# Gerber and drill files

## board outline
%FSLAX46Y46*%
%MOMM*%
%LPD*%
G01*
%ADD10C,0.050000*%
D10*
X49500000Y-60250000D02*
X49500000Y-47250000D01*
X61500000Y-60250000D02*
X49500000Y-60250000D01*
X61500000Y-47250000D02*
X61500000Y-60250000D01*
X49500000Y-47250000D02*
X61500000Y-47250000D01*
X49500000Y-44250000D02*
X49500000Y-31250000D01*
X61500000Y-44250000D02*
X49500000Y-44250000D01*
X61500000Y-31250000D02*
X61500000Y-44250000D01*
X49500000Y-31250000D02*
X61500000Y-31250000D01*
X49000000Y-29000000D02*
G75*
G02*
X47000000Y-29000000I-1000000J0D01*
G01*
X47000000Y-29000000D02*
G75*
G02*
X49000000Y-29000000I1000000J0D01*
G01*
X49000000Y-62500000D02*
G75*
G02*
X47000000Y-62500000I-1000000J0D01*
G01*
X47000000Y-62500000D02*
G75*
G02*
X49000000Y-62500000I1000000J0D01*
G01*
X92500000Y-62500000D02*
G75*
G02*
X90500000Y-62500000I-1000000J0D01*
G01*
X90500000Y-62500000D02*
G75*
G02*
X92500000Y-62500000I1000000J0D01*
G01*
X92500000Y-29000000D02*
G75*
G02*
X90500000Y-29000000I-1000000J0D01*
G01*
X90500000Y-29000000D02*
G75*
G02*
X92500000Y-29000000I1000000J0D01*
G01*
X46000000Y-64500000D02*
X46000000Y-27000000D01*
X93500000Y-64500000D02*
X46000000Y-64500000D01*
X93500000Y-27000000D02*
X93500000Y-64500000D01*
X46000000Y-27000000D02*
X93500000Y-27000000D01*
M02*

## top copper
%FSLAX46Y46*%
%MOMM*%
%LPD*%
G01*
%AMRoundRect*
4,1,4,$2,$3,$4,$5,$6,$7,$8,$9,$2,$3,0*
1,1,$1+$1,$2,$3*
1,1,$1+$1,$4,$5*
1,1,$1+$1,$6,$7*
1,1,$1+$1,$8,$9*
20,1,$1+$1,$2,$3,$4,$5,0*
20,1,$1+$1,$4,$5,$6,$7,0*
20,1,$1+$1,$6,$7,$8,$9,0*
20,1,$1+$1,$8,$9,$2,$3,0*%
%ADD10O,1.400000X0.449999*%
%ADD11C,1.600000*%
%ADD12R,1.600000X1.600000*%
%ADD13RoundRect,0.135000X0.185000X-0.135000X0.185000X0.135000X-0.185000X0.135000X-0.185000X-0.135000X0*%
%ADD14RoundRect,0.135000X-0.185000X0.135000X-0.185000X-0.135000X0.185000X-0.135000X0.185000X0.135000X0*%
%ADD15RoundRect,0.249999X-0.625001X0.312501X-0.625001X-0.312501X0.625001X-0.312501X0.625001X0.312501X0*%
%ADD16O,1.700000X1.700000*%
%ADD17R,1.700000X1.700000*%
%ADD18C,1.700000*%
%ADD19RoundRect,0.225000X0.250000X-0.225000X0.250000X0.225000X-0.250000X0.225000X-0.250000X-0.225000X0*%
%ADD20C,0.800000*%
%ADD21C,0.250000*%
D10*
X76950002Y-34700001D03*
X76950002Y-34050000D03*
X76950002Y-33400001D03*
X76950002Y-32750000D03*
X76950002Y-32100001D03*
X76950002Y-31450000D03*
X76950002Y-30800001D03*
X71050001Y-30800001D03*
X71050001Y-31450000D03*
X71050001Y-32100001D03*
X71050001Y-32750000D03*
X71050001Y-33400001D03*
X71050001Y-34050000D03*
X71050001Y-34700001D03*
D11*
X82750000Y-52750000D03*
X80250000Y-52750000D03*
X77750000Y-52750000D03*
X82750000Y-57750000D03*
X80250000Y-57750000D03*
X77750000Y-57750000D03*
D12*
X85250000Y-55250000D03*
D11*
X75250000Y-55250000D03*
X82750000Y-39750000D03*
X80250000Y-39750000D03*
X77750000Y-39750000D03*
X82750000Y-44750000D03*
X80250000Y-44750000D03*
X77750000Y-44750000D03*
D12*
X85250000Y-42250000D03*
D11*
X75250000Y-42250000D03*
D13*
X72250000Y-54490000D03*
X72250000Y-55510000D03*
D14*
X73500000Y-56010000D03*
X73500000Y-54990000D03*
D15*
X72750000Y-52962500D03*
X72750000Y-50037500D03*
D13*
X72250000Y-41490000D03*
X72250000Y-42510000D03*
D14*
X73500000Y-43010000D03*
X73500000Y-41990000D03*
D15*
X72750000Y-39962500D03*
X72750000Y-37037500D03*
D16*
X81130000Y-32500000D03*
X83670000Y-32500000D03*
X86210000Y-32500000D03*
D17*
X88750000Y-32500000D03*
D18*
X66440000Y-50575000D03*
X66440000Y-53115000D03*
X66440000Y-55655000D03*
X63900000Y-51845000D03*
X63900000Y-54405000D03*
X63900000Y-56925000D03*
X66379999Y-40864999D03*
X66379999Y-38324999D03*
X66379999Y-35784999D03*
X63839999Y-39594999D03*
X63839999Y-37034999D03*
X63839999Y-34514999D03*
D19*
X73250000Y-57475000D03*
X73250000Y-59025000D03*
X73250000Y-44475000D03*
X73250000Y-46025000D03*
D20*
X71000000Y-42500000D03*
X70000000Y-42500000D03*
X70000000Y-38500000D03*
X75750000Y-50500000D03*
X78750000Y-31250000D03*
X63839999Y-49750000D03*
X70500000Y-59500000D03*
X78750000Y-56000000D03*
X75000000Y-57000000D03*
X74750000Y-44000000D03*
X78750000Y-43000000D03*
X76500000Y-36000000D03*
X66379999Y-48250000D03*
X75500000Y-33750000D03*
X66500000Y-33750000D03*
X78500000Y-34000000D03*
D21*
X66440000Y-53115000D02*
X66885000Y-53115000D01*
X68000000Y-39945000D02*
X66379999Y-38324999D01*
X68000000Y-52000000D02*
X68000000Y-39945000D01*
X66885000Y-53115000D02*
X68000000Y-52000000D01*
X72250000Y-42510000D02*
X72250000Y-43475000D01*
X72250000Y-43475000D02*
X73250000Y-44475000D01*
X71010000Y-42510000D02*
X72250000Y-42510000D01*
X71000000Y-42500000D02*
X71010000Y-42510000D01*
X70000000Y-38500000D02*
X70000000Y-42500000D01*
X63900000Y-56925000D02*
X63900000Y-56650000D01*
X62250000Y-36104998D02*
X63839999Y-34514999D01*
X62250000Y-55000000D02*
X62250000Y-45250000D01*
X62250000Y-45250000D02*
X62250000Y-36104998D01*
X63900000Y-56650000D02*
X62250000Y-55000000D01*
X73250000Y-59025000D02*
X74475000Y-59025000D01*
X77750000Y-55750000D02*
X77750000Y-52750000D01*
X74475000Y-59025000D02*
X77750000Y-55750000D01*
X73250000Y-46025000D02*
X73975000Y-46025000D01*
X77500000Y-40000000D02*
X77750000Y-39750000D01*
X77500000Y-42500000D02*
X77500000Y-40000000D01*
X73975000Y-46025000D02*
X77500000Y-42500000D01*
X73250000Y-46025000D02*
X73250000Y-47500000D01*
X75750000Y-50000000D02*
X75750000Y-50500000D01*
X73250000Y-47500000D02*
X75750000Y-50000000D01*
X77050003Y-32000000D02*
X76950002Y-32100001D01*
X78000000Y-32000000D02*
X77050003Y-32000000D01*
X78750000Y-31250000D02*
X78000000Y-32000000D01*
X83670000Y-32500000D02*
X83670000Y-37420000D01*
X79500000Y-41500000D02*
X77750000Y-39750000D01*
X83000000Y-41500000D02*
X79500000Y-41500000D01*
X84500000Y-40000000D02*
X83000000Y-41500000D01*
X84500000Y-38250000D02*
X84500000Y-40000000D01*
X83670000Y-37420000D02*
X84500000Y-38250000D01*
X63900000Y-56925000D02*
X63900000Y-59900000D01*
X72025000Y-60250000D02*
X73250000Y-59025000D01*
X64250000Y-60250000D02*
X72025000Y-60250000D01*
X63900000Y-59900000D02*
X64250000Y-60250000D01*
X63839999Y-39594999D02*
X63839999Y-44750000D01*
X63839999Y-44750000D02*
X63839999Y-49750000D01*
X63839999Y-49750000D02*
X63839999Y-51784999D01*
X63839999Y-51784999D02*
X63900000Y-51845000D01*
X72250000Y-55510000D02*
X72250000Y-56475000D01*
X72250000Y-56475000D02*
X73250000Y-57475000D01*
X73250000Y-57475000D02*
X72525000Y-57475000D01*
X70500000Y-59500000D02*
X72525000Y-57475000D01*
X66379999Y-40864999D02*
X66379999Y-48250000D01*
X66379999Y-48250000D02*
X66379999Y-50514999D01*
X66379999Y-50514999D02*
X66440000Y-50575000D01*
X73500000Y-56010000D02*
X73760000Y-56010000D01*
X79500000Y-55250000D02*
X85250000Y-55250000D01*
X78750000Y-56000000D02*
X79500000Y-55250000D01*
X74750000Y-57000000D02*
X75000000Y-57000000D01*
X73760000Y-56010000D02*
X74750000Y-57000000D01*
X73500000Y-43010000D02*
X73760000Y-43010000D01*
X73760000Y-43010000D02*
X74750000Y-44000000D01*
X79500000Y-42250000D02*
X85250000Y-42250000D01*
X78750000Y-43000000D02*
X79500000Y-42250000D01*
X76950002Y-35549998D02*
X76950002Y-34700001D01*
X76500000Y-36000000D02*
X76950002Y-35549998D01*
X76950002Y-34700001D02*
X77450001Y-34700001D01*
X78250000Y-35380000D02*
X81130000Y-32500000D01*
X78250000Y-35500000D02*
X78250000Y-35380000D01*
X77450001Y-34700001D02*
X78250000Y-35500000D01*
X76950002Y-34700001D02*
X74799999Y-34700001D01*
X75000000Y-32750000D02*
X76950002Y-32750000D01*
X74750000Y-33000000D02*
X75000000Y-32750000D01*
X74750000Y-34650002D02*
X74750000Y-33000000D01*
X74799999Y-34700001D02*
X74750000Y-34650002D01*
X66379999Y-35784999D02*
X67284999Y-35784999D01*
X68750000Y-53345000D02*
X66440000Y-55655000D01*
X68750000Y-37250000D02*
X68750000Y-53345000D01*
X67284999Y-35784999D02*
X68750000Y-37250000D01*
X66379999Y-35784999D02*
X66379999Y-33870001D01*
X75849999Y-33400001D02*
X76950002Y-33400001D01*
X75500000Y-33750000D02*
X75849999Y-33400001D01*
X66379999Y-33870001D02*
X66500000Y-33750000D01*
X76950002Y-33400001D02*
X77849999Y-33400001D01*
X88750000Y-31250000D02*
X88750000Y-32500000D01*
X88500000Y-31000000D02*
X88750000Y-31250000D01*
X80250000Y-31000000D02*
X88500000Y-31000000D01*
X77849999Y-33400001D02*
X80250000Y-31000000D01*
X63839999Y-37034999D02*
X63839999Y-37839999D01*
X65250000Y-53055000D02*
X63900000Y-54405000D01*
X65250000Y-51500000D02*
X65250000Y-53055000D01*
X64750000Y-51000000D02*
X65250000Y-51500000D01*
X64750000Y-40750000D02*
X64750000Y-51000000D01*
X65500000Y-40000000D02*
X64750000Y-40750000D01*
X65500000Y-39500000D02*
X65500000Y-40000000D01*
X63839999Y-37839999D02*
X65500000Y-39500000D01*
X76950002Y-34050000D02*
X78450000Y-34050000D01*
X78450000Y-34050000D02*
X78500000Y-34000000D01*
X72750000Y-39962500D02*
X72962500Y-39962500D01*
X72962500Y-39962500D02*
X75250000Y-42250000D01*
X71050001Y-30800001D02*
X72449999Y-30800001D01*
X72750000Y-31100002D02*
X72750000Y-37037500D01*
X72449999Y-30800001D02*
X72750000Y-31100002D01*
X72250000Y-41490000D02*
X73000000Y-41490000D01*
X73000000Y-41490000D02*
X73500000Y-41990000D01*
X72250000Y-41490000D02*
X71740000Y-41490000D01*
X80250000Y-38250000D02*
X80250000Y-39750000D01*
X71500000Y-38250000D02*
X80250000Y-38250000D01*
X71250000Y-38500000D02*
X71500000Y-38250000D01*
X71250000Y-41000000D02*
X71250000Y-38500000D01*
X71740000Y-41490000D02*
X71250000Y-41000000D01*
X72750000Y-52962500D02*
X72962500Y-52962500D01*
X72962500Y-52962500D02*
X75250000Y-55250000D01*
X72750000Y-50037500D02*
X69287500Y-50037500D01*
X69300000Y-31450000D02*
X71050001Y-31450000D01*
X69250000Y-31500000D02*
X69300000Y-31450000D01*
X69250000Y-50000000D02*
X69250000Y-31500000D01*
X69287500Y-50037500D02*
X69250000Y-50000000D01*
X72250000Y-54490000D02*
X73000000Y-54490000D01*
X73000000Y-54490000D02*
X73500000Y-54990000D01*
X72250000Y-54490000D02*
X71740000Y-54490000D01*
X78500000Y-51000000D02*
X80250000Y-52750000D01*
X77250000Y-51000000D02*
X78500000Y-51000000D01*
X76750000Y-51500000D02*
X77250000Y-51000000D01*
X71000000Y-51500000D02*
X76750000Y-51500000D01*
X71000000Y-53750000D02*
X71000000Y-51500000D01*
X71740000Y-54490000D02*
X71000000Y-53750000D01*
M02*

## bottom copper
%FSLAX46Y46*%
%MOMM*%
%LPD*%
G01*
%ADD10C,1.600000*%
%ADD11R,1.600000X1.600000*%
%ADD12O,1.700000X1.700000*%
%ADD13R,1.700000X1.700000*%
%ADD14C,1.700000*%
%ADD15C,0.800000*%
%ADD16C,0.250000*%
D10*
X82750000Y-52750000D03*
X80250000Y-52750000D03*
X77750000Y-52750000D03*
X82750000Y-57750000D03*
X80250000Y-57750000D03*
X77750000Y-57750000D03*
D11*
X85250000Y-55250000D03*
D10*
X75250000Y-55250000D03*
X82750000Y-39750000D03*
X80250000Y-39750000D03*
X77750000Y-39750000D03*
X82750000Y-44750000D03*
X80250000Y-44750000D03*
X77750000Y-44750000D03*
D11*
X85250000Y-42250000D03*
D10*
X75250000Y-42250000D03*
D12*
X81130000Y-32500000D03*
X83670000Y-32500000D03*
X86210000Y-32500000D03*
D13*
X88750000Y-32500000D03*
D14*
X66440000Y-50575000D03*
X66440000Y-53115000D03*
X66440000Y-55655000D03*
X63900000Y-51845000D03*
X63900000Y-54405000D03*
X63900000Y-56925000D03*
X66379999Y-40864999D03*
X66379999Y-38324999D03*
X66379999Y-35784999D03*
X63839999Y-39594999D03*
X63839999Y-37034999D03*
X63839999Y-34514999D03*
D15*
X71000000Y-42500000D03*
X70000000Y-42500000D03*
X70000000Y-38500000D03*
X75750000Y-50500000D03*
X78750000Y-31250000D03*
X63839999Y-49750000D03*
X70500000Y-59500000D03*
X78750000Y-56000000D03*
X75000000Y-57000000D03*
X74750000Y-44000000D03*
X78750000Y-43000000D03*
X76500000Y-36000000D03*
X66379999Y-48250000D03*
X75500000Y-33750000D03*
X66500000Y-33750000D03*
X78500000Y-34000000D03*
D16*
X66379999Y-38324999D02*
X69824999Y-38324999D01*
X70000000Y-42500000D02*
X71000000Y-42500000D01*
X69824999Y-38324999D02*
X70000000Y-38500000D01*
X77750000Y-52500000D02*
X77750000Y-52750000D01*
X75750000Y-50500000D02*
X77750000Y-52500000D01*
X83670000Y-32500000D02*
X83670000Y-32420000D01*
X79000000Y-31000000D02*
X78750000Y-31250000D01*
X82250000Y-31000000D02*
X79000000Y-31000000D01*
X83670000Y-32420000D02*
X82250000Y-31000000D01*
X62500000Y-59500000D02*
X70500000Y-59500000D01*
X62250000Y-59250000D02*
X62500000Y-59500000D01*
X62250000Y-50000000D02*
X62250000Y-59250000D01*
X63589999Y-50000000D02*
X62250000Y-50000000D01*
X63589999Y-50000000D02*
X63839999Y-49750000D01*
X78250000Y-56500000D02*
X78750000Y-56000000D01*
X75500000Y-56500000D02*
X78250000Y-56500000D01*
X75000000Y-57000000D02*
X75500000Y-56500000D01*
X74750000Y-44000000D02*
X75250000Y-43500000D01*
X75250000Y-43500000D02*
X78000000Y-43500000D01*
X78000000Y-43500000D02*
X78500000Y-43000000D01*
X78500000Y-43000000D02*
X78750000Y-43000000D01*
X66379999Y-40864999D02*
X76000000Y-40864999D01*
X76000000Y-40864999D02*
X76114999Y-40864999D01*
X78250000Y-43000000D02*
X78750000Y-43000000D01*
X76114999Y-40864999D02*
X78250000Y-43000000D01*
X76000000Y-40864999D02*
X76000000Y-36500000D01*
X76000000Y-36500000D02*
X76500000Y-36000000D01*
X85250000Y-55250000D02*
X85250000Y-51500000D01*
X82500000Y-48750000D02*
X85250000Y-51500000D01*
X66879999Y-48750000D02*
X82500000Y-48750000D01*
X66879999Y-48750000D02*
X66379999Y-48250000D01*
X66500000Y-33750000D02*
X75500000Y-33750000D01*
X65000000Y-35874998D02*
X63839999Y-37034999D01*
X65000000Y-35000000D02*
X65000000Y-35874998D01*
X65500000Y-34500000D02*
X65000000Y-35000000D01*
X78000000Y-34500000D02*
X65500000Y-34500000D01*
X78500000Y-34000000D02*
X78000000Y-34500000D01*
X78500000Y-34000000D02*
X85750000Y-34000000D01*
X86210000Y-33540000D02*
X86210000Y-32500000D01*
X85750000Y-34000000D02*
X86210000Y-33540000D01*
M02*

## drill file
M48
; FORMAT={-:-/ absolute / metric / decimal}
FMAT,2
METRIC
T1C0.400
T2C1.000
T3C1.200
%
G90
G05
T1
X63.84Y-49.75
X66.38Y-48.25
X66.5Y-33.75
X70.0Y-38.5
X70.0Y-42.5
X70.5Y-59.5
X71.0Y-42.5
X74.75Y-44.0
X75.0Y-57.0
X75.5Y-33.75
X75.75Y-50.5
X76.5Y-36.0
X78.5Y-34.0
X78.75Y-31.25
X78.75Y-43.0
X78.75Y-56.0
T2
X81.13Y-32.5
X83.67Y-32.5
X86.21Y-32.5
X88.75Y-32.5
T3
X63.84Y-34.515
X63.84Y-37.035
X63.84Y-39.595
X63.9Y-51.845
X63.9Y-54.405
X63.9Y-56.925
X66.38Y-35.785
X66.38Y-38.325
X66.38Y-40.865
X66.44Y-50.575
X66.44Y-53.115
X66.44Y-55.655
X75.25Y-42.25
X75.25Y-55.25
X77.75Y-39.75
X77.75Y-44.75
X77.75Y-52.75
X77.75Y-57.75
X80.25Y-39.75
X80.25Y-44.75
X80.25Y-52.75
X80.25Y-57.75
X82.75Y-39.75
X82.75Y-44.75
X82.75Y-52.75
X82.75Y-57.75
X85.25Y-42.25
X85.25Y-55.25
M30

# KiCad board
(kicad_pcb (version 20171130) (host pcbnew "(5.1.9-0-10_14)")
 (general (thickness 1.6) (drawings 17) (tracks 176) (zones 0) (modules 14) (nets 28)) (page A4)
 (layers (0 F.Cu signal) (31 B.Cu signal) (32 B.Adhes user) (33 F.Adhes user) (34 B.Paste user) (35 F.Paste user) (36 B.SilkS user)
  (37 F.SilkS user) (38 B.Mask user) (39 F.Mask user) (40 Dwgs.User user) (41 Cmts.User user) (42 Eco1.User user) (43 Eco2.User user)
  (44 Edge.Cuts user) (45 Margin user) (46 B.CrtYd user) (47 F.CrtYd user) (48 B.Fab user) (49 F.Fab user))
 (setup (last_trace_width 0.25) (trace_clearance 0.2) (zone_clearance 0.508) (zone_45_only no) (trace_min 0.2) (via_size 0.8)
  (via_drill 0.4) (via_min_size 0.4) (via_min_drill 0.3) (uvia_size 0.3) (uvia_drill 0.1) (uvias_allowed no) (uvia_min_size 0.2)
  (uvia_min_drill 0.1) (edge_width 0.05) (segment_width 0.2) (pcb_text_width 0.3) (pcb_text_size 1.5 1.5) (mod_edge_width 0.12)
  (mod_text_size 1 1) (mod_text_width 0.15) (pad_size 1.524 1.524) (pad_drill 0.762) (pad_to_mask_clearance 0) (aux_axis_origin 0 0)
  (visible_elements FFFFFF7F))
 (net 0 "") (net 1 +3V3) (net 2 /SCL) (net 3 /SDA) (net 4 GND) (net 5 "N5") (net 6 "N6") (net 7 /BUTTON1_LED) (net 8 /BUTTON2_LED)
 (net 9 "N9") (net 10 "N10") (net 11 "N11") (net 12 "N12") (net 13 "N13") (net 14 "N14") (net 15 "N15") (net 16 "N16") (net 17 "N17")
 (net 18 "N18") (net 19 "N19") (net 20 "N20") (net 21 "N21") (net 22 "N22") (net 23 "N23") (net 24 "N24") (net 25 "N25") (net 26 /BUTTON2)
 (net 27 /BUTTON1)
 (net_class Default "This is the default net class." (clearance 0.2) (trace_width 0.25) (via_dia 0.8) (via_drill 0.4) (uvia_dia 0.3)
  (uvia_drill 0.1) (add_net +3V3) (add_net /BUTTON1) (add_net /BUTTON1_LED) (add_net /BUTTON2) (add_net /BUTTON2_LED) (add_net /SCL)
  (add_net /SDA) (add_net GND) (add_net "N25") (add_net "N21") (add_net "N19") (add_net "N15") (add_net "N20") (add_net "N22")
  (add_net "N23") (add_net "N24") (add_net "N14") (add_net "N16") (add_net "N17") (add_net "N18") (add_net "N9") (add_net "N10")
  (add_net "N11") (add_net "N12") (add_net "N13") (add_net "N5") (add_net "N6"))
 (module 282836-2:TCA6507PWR (layer F.Cu) (at 74 32.75 180)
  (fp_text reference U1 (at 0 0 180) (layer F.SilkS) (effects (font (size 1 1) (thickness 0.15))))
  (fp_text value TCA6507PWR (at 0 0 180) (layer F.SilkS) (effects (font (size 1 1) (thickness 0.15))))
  (pad 1 smd oval (at -2.950002 -1.950001 270) (size 0.449999 1.4) (layers F.Cu F.Paste F.Mask) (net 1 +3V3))
  (pad 2 smd oval (at -2.950002 -1.3 270) (size 0.449999 1.4) (layers F.Cu F.Paste F.Mask) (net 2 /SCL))
  (pad 3 smd oval (at -2.950002 -0.650001 270) (size 0.449999 1.4) (layers F.Cu F.Paste F.Mask) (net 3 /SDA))
  (pad 4 smd oval (at -2.950002 0 270) (size 0.449999 1.4) (layers F.Cu F.Paste F.Mask) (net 1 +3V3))
  (pad 5 smd oval (at -2.950002 0.649999 270) (size 0.449999 1.4) (layers F.Cu F.Paste F.Mask) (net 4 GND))
  (pad 6 smd oval (at -2.950002 1.3 270) (size 0.449999 1.4) (layers F.Cu F.Paste F.Mask) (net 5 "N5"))
  (pad 7 smd oval (at -2.950002 1.949999 270) (size 0.449999 1.4) (layers F.Cu F.Paste F.Mask) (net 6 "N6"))
  (pad 8 smd oval (at 2.949999 1.949999 270) (size 0.449999 1.4) (layers F.Cu F.Paste F.Mask) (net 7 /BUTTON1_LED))
  (pad 9 smd oval (at 2.949999 1.3 270) (size 0.449999 1.4) (layers F.Cu F.Paste F.Mask) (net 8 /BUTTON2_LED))
  (pad 10 smd oval (at 2.949999 0.649999 270) (size 0.449999 1.4) (layers F.Cu F.Paste F.Mask) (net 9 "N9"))
  (pad 11 smd oval (at 2.949999 0 270) (size 0.449999 1.4) (layers F.Cu F.Paste F.Mask) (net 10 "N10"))
  (pad 12 smd oval (at 2.949999 -0.650001 270) (size 0.449999 1.4) (layers F.Cu F.Paste F.Mask) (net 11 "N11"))
  (pad 13 smd oval (at 2.949999 -1.3 270) (size 0.449999 1.4) (layers F.Cu F.Paste F.Mask) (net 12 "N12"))
  (pad 14 smd oval (at 2.949999 -1.950001 270) (size 0.449999 1.4) (layers F.Cu F.Paste F.Mask) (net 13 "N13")))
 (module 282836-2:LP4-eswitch (layer F.Cu) (at 80.25 55.25)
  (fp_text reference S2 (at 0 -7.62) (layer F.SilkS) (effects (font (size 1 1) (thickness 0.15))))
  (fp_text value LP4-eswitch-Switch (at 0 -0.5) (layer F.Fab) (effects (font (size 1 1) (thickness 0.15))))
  (pad 1 thru_hole circle (at 2.5 -2.5) (size 1.6 1.6) (drill 1.2) (layers *.Cu *.Mask) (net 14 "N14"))
  (pad 2 thru_hole circle (at 0 -2.5) (size 1.6 1.6) (drill 1.2) (layers *.Cu *.Mask) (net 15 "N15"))
  (pad 3 thru_hole circle (at -2.5 -2.5) (size 1.6 1.6) (drill 1.2) (layers *.Cu *.Mask) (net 4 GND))
  (pad 4 thru_hole circle (at 2.5 2.5) (size 1.6 1.6) (drill 1.2) (layers *.Cu *.Mask) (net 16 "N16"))
  (pad 5 thru_hole circle (at 0 2.5) (size 1.6 1.6) (drill 1.2) (layers *.Cu *.Mask) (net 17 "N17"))
  (pad 6 thru_hole circle (at -2.5 2.5) (size 1.6 1.6) (drill 1.2) (layers *.Cu *.Mask) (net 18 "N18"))
  (pad L1 thru_hole rect (at 5 0) (size 1.6 1.6) (drill 1.2) (layers *.Cu *.Mask) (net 1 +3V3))
  (pad L2 thru_hole circle (at -5 0) (size 1.6 1.6) (drill 1.2) (layers *.Cu *.Mask) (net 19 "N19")))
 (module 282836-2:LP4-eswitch (layer F.Cu) (at 80.25 42.25)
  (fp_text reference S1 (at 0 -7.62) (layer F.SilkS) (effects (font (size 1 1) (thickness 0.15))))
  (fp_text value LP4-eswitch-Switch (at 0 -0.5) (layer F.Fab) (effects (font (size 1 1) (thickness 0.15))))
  (pad 1 thru_hole circle (at 2.5 -2.5) (size 1.6 1.6) (drill 1.2) (layers *.Cu *.Mask) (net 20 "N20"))
  (pad 2 thru_hole circle (at 0 -2.5) (size 1.6 1.6) (drill 1.2) (layers *.Cu *.Mask) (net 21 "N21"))
  (pad 3 thru_hole circle (at -2.5 -2.5) (size 1.6 1.6) (drill 1.2) (layers *.Cu *.Mask) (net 4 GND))
  (pad 4 thru_hole circle (at 2.5 2.5) (size 1.6 1.6) (drill 1.2) (layers *.Cu *.Mask) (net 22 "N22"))
  (pad 5 thru_hole circle (at 0 2.5) (size 1.6 1.6) (drill 1.2) (layers *.Cu *.Mask) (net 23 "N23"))
  (pad 6 thru_hole circle (at -2.5 2.5) (size 1.6 1.6) (drill 1.2) (layers *.Cu *.Mask) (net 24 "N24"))
  (pad L1 thru_hole rect (at 5 0) (size 1.6 1.6) (drill 1.2) (layers *.Cu *.Mask) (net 1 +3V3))
  (pad L2 thru_hole circle (at -5 0) (size 1.6 1.6) (drill 1.2) (layers *.Cu *.Mask) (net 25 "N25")))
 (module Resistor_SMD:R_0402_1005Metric (layer F.Cu) (at 72.25 55 90)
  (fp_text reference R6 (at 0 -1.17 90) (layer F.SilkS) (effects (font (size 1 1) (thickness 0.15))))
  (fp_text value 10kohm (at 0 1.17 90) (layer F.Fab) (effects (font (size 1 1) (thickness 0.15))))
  (pad 2 smd roundrect (at 0.51 0 90) (size 0.54 0.64) (layers F.Cu F.Paste F.Mask) (roundrect_rratio 0.25) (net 15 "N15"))
  (pad 1 smd roundrect (at -0.51 0 90) (size 0.54 0.64) (layers F.Cu F.Paste F.Mask) (roundrect_rratio 0.25) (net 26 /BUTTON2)))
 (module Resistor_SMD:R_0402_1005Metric (layer F.Cu) (at 73.5 55.5 270)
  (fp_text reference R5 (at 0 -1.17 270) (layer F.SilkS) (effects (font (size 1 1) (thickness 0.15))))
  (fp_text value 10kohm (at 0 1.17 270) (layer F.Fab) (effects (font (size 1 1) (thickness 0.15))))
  (pad 2 smd roundrect (at 0.51 0 270) (size 0.54 0.64) (layers F.Cu F.Paste F.Mask) (roundrect_rratio 0.25) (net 1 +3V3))
  (pad 1 smd roundrect (at -0.51 0 270) (size 0.54 0.64) (layers F.Cu F.Paste F.Mask) (roundrect_rratio 0.25) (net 15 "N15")))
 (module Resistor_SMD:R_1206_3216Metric (layer F.Cu) (at 72.75 51.5 270)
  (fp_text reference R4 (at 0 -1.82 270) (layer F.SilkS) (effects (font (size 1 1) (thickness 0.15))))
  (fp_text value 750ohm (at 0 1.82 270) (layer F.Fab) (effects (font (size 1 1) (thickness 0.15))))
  (pad 2 smd roundrect (at 1.4625 0 270) (size 1.125 1.75) (layers F.Cu F.Paste F.Mask) (roundrect_rratio 0.2222213333333333) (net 19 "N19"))
  (pad 1 smd roundrect (at -1.4625 0 270) (size 1.125 1.75) (layers F.Cu F.Paste F.Mask) (roundrect_rratio 0.2222213333333333)
   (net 8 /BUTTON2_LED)))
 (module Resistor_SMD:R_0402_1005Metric (layer F.Cu) (at 72.25 42 90)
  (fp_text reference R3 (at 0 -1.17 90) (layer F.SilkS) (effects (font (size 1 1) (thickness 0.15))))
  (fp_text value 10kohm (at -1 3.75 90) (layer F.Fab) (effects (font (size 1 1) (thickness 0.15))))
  (pad 2 smd roundrect (at 0.51 0 90) (size 0.54 0.64) (layers F.Cu F.Paste F.Mask) (roundrect_rratio 0.25) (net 21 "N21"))
  (pad 1 smd roundrect (at -0.51 0 90) (size 0.54 0.64) (layers F.Cu F.Paste F.Mask) (roundrect_rratio 0.25) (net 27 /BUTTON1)))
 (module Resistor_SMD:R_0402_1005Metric (layer F.Cu) (at 73.5 42.5 270)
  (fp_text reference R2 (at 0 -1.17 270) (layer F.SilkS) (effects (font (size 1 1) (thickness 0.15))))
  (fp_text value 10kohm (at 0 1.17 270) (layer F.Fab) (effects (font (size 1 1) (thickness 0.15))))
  (pad 2 smd roundrect (at 0.51 0 270) (size 0.54 0.64) (layers F.Cu F.Paste F.Mask) (roundrect_rratio 0.25) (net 1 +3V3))
  (pad 1 smd roundrect (at -0.51 0 270) (size 0.54 0.64) (layers F.Cu F.Paste F.Mask) (roundrect_rratio 0.25) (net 21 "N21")))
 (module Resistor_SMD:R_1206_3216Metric (layer F.Cu) (at 72.75 38.5 270)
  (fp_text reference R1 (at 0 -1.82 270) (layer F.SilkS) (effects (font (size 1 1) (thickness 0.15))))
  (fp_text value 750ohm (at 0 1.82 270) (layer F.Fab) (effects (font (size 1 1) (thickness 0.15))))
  (pad 2 smd roundrect (at 1.4625 0 270) (size 1.125 1.75) (layers F.Cu F.Paste F.Mask) (roundrect_rratio 0.2222213333333333) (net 25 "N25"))
  (pad 1 smd roundrect (at -1.4625 0 270) (size 1.125 1.75) (layers F.Cu F.Paste F.Mask) (roundrect_rratio 0.2222213333333333)
   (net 7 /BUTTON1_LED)))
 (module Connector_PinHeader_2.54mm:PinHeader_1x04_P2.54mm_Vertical (layer F.Cu) (at 88.75 32.5 270)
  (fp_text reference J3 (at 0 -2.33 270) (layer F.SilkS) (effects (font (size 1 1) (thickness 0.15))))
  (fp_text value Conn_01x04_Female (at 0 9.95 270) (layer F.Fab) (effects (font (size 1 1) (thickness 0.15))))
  (pad 4 thru_hole oval (at 0 7.62 270) (size 1.7 1.7) (drill 1) (layers *.Cu *.Mask) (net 1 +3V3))
  (pad 3 thru_hole oval (at 0 5.08 270) (size 1.7 1.7) (drill 1) (layers *.Cu *.Mask) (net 4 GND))
  (pad 2 thru_hole oval (at 0 2.54 270) (size 1.7 1.7) (drill 1) (layers *.Cu *.Mask) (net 2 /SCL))
  (pad 1 thru_hole rect (at 0 0 270) (size 1.7 1.7) (drill 1) (layers *.Cu *.Mask) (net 3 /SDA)))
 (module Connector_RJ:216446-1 (layer B.Cu) (at 61.5 53.75 90)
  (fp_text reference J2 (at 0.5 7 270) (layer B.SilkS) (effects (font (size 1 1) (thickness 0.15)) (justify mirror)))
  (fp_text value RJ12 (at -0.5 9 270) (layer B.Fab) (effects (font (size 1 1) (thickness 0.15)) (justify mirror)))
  (pad 6 thru_hole circle (at 3.175 4.94 90) (size 1.7 1.7) (drill 1.2) (layers *.Cu *.Mask) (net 1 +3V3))
  (pad 4 thru_hole circle (at 0.635 4.94 90) (size 1.7 1.7) (drill 1.2) (layers *.Cu *.Mask) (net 27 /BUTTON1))
  (pad 2 thru_hole circle (at -1.905 4.94 90) (size 1.7 1.7) (drill 1.2) (layers *.Cu *.Mask) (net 3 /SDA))
  (pad 5 thru_hole circle (at 1.905 2.4 90) (size 1.7 1.7) (drill 1.2) (layers *.Cu *.Mask) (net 26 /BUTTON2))
  (pad 3 thru_hole circle (at -0.655 2.4 90) (size 1.7 1.7) (drill 1.2) (layers *.Cu *.Mask) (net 2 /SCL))
  (pad 1 thru_hole circle (at -3.175 2.4 90) (size 1.7 1.7) (drill 1.2) (layers *.Cu *.Mask) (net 4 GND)))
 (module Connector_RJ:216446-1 (layer F.Cu) (at 61.439999 37.689999 270)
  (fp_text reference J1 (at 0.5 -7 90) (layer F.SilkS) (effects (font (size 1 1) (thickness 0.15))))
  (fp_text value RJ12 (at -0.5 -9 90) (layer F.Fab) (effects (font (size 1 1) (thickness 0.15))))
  (pad 6 thru_hole circle (at 3.175 -4.94 270) (size 1.7 1.7) (drill 1.2) (layers *.Cu *.Mask) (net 1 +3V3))
  (pad 4 thru_hole circle (at 0.635 -4.94 270) (size 1.7 1.7) (drill 1.2) (layers *.Cu *.Mask) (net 27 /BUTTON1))
  (pad 2 thru_hole circle (at -1.905 -4.94 270) (size 1.7 1.7) (drill 1.2) (layers *.Cu *.Mask) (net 3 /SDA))
  (pad 5 thru_hole circle (at 1.905 -2.4 270) (size 1.7 1.7) (drill 1.2) (layers *.Cu *.Mask) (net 26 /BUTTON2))
  (pad 3 thru_hole circle (at -0.655 -2.4 270) (size 1.7 1.7) (drill 1.2) (layers *.Cu *.Mask) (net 2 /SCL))
  (pad 1 thru_hole circle (at -3.175 -2.4 270) (size 1.7 1.7) (drill 1.2) (layers *.Cu *.Mask) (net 4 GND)))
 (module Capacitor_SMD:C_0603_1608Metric (layer F.Cu) (at 73.25 58.25 90)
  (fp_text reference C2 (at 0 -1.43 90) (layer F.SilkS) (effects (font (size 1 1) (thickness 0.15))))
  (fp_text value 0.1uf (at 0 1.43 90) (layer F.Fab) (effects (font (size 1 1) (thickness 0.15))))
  (pad 2 smd roundrect (at 0.775 0 90) (size 0.9 0.95) (layers F.Cu F.Paste F.Mask) (roundrect_rratio 0.25) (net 26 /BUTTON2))
  (pad 1 smd roundrect (at -0.775 0 90) (size 0.9 0.95) (layers F.Cu F.Paste F.Mask) (roundrect_rratio 0.25) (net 4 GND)))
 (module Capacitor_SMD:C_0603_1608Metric (layer F.Cu) (at 73.25 45.25 90)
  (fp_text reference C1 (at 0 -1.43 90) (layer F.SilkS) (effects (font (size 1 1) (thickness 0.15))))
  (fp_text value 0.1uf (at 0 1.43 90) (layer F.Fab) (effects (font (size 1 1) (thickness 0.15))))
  (pad 2 smd roundrect (at 0.775 0 90) (size 0.9 0.95) (layers F.Cu F.Paste F.Mask) (roundrect_rratio 0.25) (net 27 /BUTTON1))
  (pad 1 smd roundrect (at -0.775 0 90) (size 0.9 0.95) (layers F.Cu F.Paste F.Mask) (roundrect_rratio 0.25) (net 4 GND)))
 (gr_line (start 49.5 60.25) (end 49.5 47.25) (angle 90) (layer Edge.Cuts) (width 0.05))
 (gr_line (start 61.5 60.25) (end 49.5 60.25) (angle 90) (layer Edge.Cuts) (width 0.05))
 (gr_line (start 61.5 47.25) (end 61.5 60.25) (angle 90) (layer Edge.Cuts) (width 0.05))
 (gr_line (start 49.5 47.25) (end 61.5 47.25) (angle 90) (layer Edge.Cuts) (width 0.05))
 (gr_line (start 49.5 44.25) (end 49.5 31.25) (angle 90) (layer Edge.Cuts) (width 0.05))
 (gr_line (start 61.5 44.25) (end 49.5 44.25) (angle 90) (layer Edge.Cuts) (width 0.05))
 (gr_line (start 61.5 31.25) (end 61.5 44.25) (angle 90) (layer Edge.Cuts) (width 0.05))
 (gr_line (start 49.5 31.25) (end 61.5 31.25) (angle 90) (layer Edge.Cuts) (width 0.05))
 (gr_circle (center 48 29) (end 49 29) (layer Edge.Cuts) (width 0.05))
 (gr_circle (center 48 62.5) (end 49 62.5) (layer Edge.Cuts) (width 0.05))
 (gr_circle (center 91.5 62.5) (end 92.5 62.5) (layer Edge.Cuts) (width 0.05))
 (gr_circle (center 91.5 29) (end 92.5 29) (layer Edge.Cuts) (width 0.05))
 (gr_line (start 46 64.5) (end 46 27) (angle 90) (layer Edge.Cuts) (width 0.05))
 (gr_line (start 93.5 64.5) (end 46 64.5) (angle 90) (layer Edge.Cuts) (width 0.05))
 (gr_line (start 93.5 27) (end 93.5 64.5) (angle 90) (layer Edge.Cuts) (width 0.05))
 (gr_line (start 46 27) (end 93.5 27) (angle 90) (layer Edge.Cuts) (width 0.05))
 (segment (start 66.44 53.115) (end 66.885 53.115) (width 0.25) (layer F.Cu) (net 27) (status C00000))
 (segment (start 68 39.945) (end 66.379999 38.324999) (width 0.25) (layer F.Cu) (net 27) (status 800000))
 (segment (start 68 52) (end 68 39.945) (width 0.25) (layer F.Cu) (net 27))
 (segment (start 66.885 53.115) (end 68 52) (width 0.25) (layer F.Cu) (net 27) (status 400000))
 (segment (start 72.25 42.51) (end 72.25 43.475) (width 0.25) (layer F.Cu) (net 27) (status 400000))
 (segment (start 72.25 43.475) (end 73.25 44.475) (width 0.25) (layer F.Cu) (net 27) (status 800000))
 (segment (start 66.379999 38.324999) (end 69.824999 38.324999) (width 0.25) (layer B.Cu) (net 27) (status 400000))
 (segment (start 71.01 42.51) (end 72.25 42.51) (width 0.25) (layer F.Cu) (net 27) (status 800000))
 (segment (start 71 42.5) (end 71.01 42.51) (width 0.25) (layer F.Cu) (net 27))
 (via (at 71 42.5) (size 0.8) (drill 0.4) (layers F.Cu B.Cu) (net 27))
 (segment (start 70 42.5) (end 71 42.5) (width 0.25) (layer B.Cu) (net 27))
 (via (at 70 42.5) (size 0.8) (drill 0.4) (layers F.Cu B.Cu) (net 27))
 (segment (start 70 38.5) (end 70 42.5) (width 0.25) (layer F.Cu) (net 27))
 (via (at 70 38.5) (size 0.8) (drill 0.4) (layers F.Cu B.Cu) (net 27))
 (segment (start 69.824999 38.324999) (end 70 38.5) (width 0.25) (layer B.Cu) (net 27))
 (segment (start 63.9 56.925) (end 63.9 56.65) (width 0.25) (layer F.Cu) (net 4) (status C00000))
 (segment (start 62.25 36.104998) (end 63.839999 34.514999) (width 0.25) (layer F.Cu) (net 4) (status 800000))
 (segment (start 62.25 55) (end 62.25 45.25) (width 0.25) (layer F.Cu) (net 4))
 (segment (start 62.25 45.25) (end 62.25 36.104998) (width 0.25) (layer F.Cu) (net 4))
 (segment (start 63.9 56.65) (end 62.25 55) (width 0.25) (layer F.Cu) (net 4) (status 400000))
 (segment (start 73.25 59.025) (end 74.475 59.025) (width 0.25) (layer F.Cu) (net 4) (status 400000))
 (segment (start 77.75 55.75) (end 77.75 52.75) (width 0.25) (layer F.Cu) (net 4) (status 800000))
 (segment (start 74.475 59.025) (end 77.75 55.75) (width 0.25) (layer F.Cu) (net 4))
 (segment (start 73.25 46.025) (end 73.975 46.025) (width 0.25) (layer F.Cu) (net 4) (status 400000))
 (segment (start 77.5 40) (end 77.75 39.75) (width 0.25) (layer F.Cu) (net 4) (status C00000))
 (segment (start 77.5 42.5) (end 77.5 40) (width 0.25) (layer F.Cu) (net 4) (status 800000))
 (segment (start 73.975 46.025) (end 77.5 42.5) (width 0.25) (layer F.Cu) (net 4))
 (segment (start 73.25 46.025) (end 73.25 47.5) (width 0.25) (layer F.Cu) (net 4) (status 400000))
 (segment (start 77.75 52.5) (end 77.75 52.75) (width 0.25) (layer B.Cu) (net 4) (status C00000))
 (segment (start 75.75 50.5) (end 77.75 52.5) (width 0.25) (layer B.Cu) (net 4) (status 800000))
 (via (at 75.75 50.5) (size 0.8) (drill 0.4) (layers F.Cu B.Cu) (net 4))
 (segment (start 75.75 50) (end 75.75 50.5) (width 0.25) (layer F.Cu) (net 4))
 (segment (start 73.25 47.5) (end 75.75 50) (width 0.25) (layer F.Cu) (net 4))
 (segment (start 83.67 32.5) (end 83.67 32.42) (width 0.25) (layer B.Cu) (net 4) (status C00000))
 (segment (start 77.050003 32) (end 76.950002 32.100001) (width 0.25) (layer F.Cu) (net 4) (status C00000))
 (segment (start 78 32) (end 77.050003 32) (width 0.25) (layer F.Cu) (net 4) (status 800000))
 (segment (start 78.75 31.25) (end 78 32) (width 0.25) (layer F.Cu) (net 4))
 (via (at 78.75 31.25) (size 0.8) (drill 0.4) (layers F.Cu B.Cu) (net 4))
 (segment (start 79 31) (end 78.75 31.25) (width 0.25) (layer B.Cu) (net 4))
 (segment (start 82.25 31) (end 79 31) (width 0.25) (layer B.Cu) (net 4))
 (segment (start 83.67 32.42) (end 82.25 31) (width 0.25) (layer B.Cu) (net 4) (status 400000))
 (segment (start 83.67 32.5) (end 83.67 37.42) (width 0.25) (layer F.Cu) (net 4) (status 400000))
 (segment (start 79.5 41.5) (end 77.75 39.75) (width 0.25) (layer F.Cu) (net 4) (status 800000))
 (segment (start 83 41.5) (end 79.5 41.5) (width 0.25) (layer F.Cu) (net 4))
 (segment (start 84.5 40) (end 83 41.5) (width 0.25) (layer F.Cu) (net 4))
 (segment (start 84.5 38.25) (end 84.5 40) (width 0.25) (layer F.Cu) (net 4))
 (segment (start 83.67 37.42) (end 84.5 38.25) (width 0.25) (layer F.Cu) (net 4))
 (segment (start 63.9 56.925) (end 63.9 59.9) (width 0.25) (layer F.Cu) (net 4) (status 400000))
 (segment (start 72.025 60.25) (end 73.25 59.025) (width 0.25) (layer F.Cu) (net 4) (status 800000))
 (segment (start 64.25 60.25) (end 72.025 60.25) (width 0.25) (layer F.Cu) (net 4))
 (segment (start 63.9 59.9) (end 64.25 60.25) (width 0.25) (layer F.Cu) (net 4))
 (segment (start 63.839999 39.594999) (end 63.839999 44.75) (width 0.25) (layer F.Cu) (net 26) (status 400000))
 (segment (start 63.839999 44.75) (end 63.839999 49.75) (width 0.25) (layer F.Cu) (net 26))
 (segment (start 63.839999 49.75) (end 63.839999 51.784999) (width 0.25) (layer F.Cu) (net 26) (status 800000))
 (segment (start 63.839999 51.784999) (end 63.9 51.845) (width 0.25) (layer F.Cu) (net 26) (status C00000))
 (segment (start 72.25 55.51) (end 72.25 56.475) (width 0.25) (layer F.Cu) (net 26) (status 400000))
 (segment (start 72.25 56.475) (end 73.25 57.475) (width 0.25) (layer F.Cu) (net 26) (status 800000))
 (via (at 63.839999 49.75) (size 0.8) (drill 0.4) (layers F.Cu B.Cu) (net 26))
 (segment (start 73.25 57.475) (end 72.525 57.475) (width 0.25) (layer F.Cu) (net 26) (status 400000))
 (segment (start 70.5 59.5) (end 72.525 57.475) (width 0.25) (layer F.Cu) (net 26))
 (via (at 70.5 59.5) (size 0.8) (drill 0.4) (layers F.Cu B.Cu) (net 26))
 (segment (start 62.5 59.5) (end 70.5 59.5) (width 0.25) (layer B.Cu) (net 26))
 (segment (start 62.25 59.25) (end 62.5 59.5) (width 0.25) (layer B.Cu) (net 26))
 (segment (start 62.25 50) (end 62.25 59.25) (width 0.25) (layer B.Cu) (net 26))
 (segment (start 63.589999 50) (end 62.25 50) (width 0.25) (layer B.Cu) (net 26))
 (segment (start 63.589999 50) (end 63.839999 49.75) (width 0.25) (layer B.Cu) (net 26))
 (segment (start 66.379999 40.864999) (end 66.379999 48.25) (width 0.25) (layer F.Cu) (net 1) (status 400000))
 (segment (start 66.379999 48.25) (end 66.379999 50.514999) (width 0.25) (layer F.Cu) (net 1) (status 800000))
 (segment (start 66.379999 50.514999) (end 66.44 50.575) (width 0.25) (layer F.Cu) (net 1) (status C00000))
 (segment (start 73.5 56.01) (end 73.76 56.01) (width 0.25) (layer F.Cu) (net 1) (status C00000))
 (segment (start 79.5 55.25) (end 85.25 55.25) (width 0.25) (layer F.Cu) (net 1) (status 800000))
 (segment (start 78.75 56) (end 79.5 55.25) (width 0.25) (layer F.Cu) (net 1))
 (via (at 78.75 56) (size 0.8) (drill 0.4) (layers F.Cu B.Cu) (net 1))
 (segment (start 78.25 56.5) (end 78.75 56) (width 0.25) (layer B.Cu) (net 1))
 (segment (start 75.5 56.5) (end 78.25 56.5) (width 0.25) (layer B.Cu) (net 1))
 (segment (start 75 57) (end 75.5 56.5) (width 0.25) (layer B.Cu) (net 1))
 (via (at 75 57) (size 0.8) (drill 0.4) (layers F.Cu B.Cu) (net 1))
 (segment (start 74.75 57) (end 75 57) (width 0.25) (layer F.Cu) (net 1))
 (segment (start 73.76 56.01) (end 74.75 57) (width 0.25) (layer F.Cu) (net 1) (status 400000))
 (segment (start 73.5 43.01) (end 73.76 43.01) (width 0.25) (layer F.Cu) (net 1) (status C00000))
 (segment (start 73.76 43.01) (end 74.75 44) (width 0.25) (layer F.Cu) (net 1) (status 400000))
 (via (at 74.75 44) (size 0.8) (drill 0.4) (layers F.Cu B.Cu) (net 1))
 (segment (start 74.75 44) (end 75.25 43.5) (width 0.25) (layer B.Cu) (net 1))
 (segment (start 75.25 43.5) (end 78 43.5) (width 0.25) (layer B.Cu) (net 1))
 (segment (start 78 43.5) (end 78.5 43) (width 0.25) (layer B.Cu) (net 1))
 (segment (start 78.5 43) (end 78.75 43) (width 0.25) (layer B.Cu) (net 1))
 (segment (start 79.5 42.25) (end 85.25 42.25) (width 0.25) (layer F.Cu) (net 1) (status 800000))
 (via (at 78.75 43) (size 0.8) (drill 0.4) (layers F.Cu B.Cu) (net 1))
 (segment (start 78.75 43) (end 79.5 42.25) (width 0.25) (layer F.Cu) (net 1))
 (segment (start 66.379999 40.864999) (end 76 40.864999) (width 0.25) (layer B.Cu) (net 1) (status 400000))
 (segment (start 76 40.864999) (end 76.114999 40.864999) (width 0.25) (layer B.Cu) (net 1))
 (segment (start 78.25 43) (end 78.75 43) (width 0.25) (layer B.Cu) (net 1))
 (segment (start 76.114999 40.864999) (end 78.25 43) (width 0.25) (layer B.Cu) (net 1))
 (segment (start 76 40.864999) (end 76 36.5) (width 0.25) (layer B.Cu) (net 1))
 (segment (start 76.950002 35.549998) (end 76.950002 34.700001) (width 0.25) (layer F.Cu) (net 1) (status 800000))
 (segment (start 76.5 36) (end 76.950002 35.549998) (width 0.25) (layer F.Cu) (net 1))
 (via (at 76.5 36) (size 0.8) (drill 0.4) (layers F.Cu B.Cu) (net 1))
 (segment (start 76 36.5) (end 76.5 36) (width 0.25) (layer B.Cu) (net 1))
 (segment (start 76.950002 34.700001) (end 77.450001 34.700001) (width 0.25) (layer F.Cu) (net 1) (status C00000))
 (segment (start 78.25 35.38) (end 81.13 32.5) (width 0.25) (layer F.Cu) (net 1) (status 800000))
 (segment (start 78.25 35.5) (end 78.25 35.38) (width 0.25) (layer F.Cu) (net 1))
 (segment (start 77.450001 34.700001) (end 78.25 35.5) (width 0.25) (layer F.Cu) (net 1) (status 400000))
 (segment (start 76.950002 34.700001) (end 74.799999 34.700001) (width 0.25) (layer F.Cu) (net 1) (status 400000))
 (segment (start 75 32.75) (end 76.950002 32.75) (width 0.25) (layer F.Cu) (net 1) (status 800000))
 (segment (start 74.75 33) (end 75 32.75) (width 0.25) (layer F.Cu) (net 1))
 (segment (start 74.75 34.650002) (end 74.75 33) (width 0.25) (layer F.Cu) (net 1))
 (segment (start 74.799999 34.700001) (end 74.75 34.650002) (width 0.25) (layer F.Cu) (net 1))
 (via (at 66.379999 48.25) (size 0.8) (drill 0.4) (layers F.Cu B.Cu) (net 1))
 (segment (start 85.25 55.25) (end 85.25 51.5) (width 0.25) (layer B.Cu) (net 1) (status 400000))
 (segment (start 82.5 48.75) (end 85.25 51.5) (width 0.25) (layer B.Cu) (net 1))
 (segment (start 66.879999 48.75) (end 82.5 48.75) (width 0.25) (layer B.Cu) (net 1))
 (segment (start 66.879999 48.75) (end 66.379999 48.25) (width 0.25) (layer B.Cu) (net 1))
 (segment (start 66.379999 35.784999) (end 67.284999 35.784999) (width 0.25) (layer F.Cu) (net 3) (status 400000))
 (segment (start 68.75 53.345) (end 66.44 55.655) (width 0.25) (layer F.Cu) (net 3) (status 800000))
 (segment (start 68.75 37.25) (end 68.75 53.345) (width 0.25) (layer F.Cu) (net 3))
 (segment (start 67.284999 35.784999) (end 68.75 37.25) (width 0.25) (layer F.Cu) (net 3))
 (segment (start 66.379999 35.784999) (end 66.379999 33.870001) (width 0.25) (layer F.Cu) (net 3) (status 400000))
 (segment (start 75.849999 33.400001) (end 76.950002 33.400001) (width 0.25) (layer F.Cu) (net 3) (status 800000))
 (segment (start 75.5 33.75) (end 75.849999 33.400001) (width 0.25) (layer F.Cu) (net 3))
 (via (at 75.5 33.75) (size 0.8) (drill 0.4) (layers F.Cu B.Cu) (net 3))
 (segment (start 66.5 33.75) (end 75.5 33.75) (width 0.25) (layer B.Cu) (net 3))
 (via (at 66.5 33.75) (size 0.8) (drill 0.4) (layers F.Cu B.Cu) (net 3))
 (segment (start 66.379999 33.870001) (end 66.5 33.75) (width 0.25) (layer F.Cu) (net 3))
 (segment (start 76.950002 33.400001) (end 77.849999 33.400001) (width 0.25) (layer F.Cu) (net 3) (status 400000))
 (segment (start 88.75 31.25) (end 88.75 32.5) (width 0.25) (layer F.Cu) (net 3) (status 800000))
 (segment (start 88.5 31) (end 88.75 31.25) (width 0.25) (layer F.Cu) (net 3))
 (segment (start 80.25 31) (end 88.5 31) (width 0.25) (layer F.Cu) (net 3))
 (segment (start 77.849999 33.400001) (end 80.25 31) (width 0.25) (layer F.Cu) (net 3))
 (segment (start 63.839999 37.034999) (end 63.839999 37.839999) (width 0.25) (layer F.Cu) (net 2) (status C00000))
 (segment (start 65.25 53.055) (end 63.9 54.405) (width 0.25) (layer F.Cu) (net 2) (status 800000))
 (segment (start 65.25 51.5) (end 65.25 53.055) (width 0.25) (layer F.Cu) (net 2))
 (segment (start 64.75 51) (end 65.25 51.5) (width 0.25) (layer F.Cu) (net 2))
 (segment (start 64.75 40.75) (end 64.75 51) (width 0.25) (layer F.Cu) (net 2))
 (segment (start 65.5 40) (end 64.75 40.75) (width 0.25) (layer F.Cu) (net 2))
 (segment (start 65.5 39.5) (end 65.5 40) (width 0.25) (layer F.Cu) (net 2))
 (segment (start 63.839999 37.839999) (end 65.5 39.5) (width 0.25) (layer F.Cu) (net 2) (status 400000))
 (segment (start 76.950002 34.05) (end 78.45 34.05) (width 0.25) (layer F.Cu) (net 2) (status 400000))
 (segment (start 65 35.874998) (end 63.839999 37.034999) (width 0.25) (layer B.Cu) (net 2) (status 800000))
 (segment (start 65 35) (end 65 35.874998) (width 0.25) (layer B.Cu) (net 2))
 (segment (start 65.5 34.5) (end 65 35) (width 0.25) (layer B.Cu) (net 2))
 (segment (start 78 34.5) (end 65.5 34.5) (width 0.25) (layer B.Cu) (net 2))
 (segment (start 78.5 34) (end 78 34.5) (width 0.25) (layer B.Cu) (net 2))
 (via (at 78.5 34) (size 0.8) (drill 0.4) (layers F.Cu B.Cu) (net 2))
 (segment (start 78.45 34.05) (end 78.5 34) (width 0.25) (layer F.Cu) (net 2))
 (segment (start 78.5 34) (end 85.75 34) (width 0.25) (layer B.Cu) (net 2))
 (segment (start 86.21 33.54) (end 86.21 32.5) (width 0.25) (layer B.Cu) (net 2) (status 800000))
 (segment (start 85.75 34) (end 86.21 33.54) (width 0.25) (layer B.Cu) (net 2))
 (segment (start 72.75 39.9625) (end 72.9625 39.9625) (width 0.25) (layer F.Cu) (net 25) (status C00000))
 (segment (start 72.9625 39.9625) (end 75.25 42.25) (width 0.25) (layer F.Cu) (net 25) (status C00000))
 (segment (start 71.050001 30.800001) (end 72.449999 30.800001) (width 0.25) (layer F.Cu) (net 7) (status 400000))
 (segment (start 72.75 31.100002) (end 72.75 37.0375) (width 0.25) (layer F.Cu) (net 7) (status 800000))
 (segment (start 72.449999 30.800001) (end 72.75 31.100002) (width 0.25) (layer F.Cu) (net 7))
 (segment (start 72.25 41.49) (end 73 41.49) (width 0.25) (layer F.Cu) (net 21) (status 400000))
 (segment (start 73 41.49) (end 73.5 41.99) (width 0.25) (layer F.Cu) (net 21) (status 800000))
 (segment (start 72.25 41.49) (end 71.74 41.49) (width 0.25) (layer F.Cu) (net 21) (status 400000))
 (segment (start 80.25 38.25) (end 80.25 39.75) (width 0.25) (layer F.Cu) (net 21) (status 800000))
 (segment (start 71.5 38.25) (end 80.25 38.25) (width 0.25) (layer F.Cu) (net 21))
 (segment (start 71.25 38.5) (end 71.5 38.25) (width 0.25) (layer F.Cu) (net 21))
 (segment (start 71.25 41) (end 71.25 38.5) (width 0.25) (layer F.Cu) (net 21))
 (segment (start 71.74 41.49) (end 71.25 41) (width 0.25) (layer F.Cu) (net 21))
 (segment (start 72.75 52.9625) (end 72.9625 52.9625) (width 0.25) (layer F.Cu) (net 19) (status C00000))
 (segment (start 72.9625 52.9625) (end 75.25 55.25) (width 0.25) (layer F.Cu) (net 19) (status C00000))
 (segment (start 72.75 50.0375) (end 69.2875 50.0375) (width 0.25) (layer F.Cu) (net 8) (status 400000))
 (segment (start 69.3 31.45) (end 71.050001 31.45) (width 0.25) (layer F.Cu) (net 8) (status 800000))
 (segment (start 69.25 31.5) (end 69.3 31.45) (width 0.25) (layer F.Cu) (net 8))
 (segment (start 69.25 50) (end 69.25 31.5) (width 0.25) (layer F.Cu) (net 8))
 (segment (start 69.2875 50.0375) (end 69.25 50) (width 0.25) (layer F.Cu) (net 8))
 (segment (start 72.25 54.49) (end 73 54.49) (width 0.25) (layer F.Cu) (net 15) (status 400000))
 (segment (start 73 54.49) (end 73.5 54.99) (width 0.25) (layer F.Cu) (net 15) (status 800000))
 (segment (start 72.25 54.49) (end 71.74 54.49) (width 0.25) (layer F.Cu) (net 15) (status 400000))
 (segment (start 78.5 51) (end 80.25 52.75) (width 0.25) (layer F.Cu) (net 15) (status 800000))
 (segment (start 77.25 51) (end 78.5 51) (width 0.25) (layer F.Cu) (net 15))
 (segment (start 76.75 51.5) (end 77.25 51) (width 0.25) (layer F.Cu) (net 15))
 (segment (start 71 51.5) (end 76.75 51.5) (width 0.25) (layer F.Cu) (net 15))
 (segment (start 71 53.75) (end 71 51.5) (width 0.25) (layer F.Cu) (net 15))
 (segment (start 71.74 54.49) (end 71 53.75) (width 0.25) (layer F.Cu) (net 15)))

